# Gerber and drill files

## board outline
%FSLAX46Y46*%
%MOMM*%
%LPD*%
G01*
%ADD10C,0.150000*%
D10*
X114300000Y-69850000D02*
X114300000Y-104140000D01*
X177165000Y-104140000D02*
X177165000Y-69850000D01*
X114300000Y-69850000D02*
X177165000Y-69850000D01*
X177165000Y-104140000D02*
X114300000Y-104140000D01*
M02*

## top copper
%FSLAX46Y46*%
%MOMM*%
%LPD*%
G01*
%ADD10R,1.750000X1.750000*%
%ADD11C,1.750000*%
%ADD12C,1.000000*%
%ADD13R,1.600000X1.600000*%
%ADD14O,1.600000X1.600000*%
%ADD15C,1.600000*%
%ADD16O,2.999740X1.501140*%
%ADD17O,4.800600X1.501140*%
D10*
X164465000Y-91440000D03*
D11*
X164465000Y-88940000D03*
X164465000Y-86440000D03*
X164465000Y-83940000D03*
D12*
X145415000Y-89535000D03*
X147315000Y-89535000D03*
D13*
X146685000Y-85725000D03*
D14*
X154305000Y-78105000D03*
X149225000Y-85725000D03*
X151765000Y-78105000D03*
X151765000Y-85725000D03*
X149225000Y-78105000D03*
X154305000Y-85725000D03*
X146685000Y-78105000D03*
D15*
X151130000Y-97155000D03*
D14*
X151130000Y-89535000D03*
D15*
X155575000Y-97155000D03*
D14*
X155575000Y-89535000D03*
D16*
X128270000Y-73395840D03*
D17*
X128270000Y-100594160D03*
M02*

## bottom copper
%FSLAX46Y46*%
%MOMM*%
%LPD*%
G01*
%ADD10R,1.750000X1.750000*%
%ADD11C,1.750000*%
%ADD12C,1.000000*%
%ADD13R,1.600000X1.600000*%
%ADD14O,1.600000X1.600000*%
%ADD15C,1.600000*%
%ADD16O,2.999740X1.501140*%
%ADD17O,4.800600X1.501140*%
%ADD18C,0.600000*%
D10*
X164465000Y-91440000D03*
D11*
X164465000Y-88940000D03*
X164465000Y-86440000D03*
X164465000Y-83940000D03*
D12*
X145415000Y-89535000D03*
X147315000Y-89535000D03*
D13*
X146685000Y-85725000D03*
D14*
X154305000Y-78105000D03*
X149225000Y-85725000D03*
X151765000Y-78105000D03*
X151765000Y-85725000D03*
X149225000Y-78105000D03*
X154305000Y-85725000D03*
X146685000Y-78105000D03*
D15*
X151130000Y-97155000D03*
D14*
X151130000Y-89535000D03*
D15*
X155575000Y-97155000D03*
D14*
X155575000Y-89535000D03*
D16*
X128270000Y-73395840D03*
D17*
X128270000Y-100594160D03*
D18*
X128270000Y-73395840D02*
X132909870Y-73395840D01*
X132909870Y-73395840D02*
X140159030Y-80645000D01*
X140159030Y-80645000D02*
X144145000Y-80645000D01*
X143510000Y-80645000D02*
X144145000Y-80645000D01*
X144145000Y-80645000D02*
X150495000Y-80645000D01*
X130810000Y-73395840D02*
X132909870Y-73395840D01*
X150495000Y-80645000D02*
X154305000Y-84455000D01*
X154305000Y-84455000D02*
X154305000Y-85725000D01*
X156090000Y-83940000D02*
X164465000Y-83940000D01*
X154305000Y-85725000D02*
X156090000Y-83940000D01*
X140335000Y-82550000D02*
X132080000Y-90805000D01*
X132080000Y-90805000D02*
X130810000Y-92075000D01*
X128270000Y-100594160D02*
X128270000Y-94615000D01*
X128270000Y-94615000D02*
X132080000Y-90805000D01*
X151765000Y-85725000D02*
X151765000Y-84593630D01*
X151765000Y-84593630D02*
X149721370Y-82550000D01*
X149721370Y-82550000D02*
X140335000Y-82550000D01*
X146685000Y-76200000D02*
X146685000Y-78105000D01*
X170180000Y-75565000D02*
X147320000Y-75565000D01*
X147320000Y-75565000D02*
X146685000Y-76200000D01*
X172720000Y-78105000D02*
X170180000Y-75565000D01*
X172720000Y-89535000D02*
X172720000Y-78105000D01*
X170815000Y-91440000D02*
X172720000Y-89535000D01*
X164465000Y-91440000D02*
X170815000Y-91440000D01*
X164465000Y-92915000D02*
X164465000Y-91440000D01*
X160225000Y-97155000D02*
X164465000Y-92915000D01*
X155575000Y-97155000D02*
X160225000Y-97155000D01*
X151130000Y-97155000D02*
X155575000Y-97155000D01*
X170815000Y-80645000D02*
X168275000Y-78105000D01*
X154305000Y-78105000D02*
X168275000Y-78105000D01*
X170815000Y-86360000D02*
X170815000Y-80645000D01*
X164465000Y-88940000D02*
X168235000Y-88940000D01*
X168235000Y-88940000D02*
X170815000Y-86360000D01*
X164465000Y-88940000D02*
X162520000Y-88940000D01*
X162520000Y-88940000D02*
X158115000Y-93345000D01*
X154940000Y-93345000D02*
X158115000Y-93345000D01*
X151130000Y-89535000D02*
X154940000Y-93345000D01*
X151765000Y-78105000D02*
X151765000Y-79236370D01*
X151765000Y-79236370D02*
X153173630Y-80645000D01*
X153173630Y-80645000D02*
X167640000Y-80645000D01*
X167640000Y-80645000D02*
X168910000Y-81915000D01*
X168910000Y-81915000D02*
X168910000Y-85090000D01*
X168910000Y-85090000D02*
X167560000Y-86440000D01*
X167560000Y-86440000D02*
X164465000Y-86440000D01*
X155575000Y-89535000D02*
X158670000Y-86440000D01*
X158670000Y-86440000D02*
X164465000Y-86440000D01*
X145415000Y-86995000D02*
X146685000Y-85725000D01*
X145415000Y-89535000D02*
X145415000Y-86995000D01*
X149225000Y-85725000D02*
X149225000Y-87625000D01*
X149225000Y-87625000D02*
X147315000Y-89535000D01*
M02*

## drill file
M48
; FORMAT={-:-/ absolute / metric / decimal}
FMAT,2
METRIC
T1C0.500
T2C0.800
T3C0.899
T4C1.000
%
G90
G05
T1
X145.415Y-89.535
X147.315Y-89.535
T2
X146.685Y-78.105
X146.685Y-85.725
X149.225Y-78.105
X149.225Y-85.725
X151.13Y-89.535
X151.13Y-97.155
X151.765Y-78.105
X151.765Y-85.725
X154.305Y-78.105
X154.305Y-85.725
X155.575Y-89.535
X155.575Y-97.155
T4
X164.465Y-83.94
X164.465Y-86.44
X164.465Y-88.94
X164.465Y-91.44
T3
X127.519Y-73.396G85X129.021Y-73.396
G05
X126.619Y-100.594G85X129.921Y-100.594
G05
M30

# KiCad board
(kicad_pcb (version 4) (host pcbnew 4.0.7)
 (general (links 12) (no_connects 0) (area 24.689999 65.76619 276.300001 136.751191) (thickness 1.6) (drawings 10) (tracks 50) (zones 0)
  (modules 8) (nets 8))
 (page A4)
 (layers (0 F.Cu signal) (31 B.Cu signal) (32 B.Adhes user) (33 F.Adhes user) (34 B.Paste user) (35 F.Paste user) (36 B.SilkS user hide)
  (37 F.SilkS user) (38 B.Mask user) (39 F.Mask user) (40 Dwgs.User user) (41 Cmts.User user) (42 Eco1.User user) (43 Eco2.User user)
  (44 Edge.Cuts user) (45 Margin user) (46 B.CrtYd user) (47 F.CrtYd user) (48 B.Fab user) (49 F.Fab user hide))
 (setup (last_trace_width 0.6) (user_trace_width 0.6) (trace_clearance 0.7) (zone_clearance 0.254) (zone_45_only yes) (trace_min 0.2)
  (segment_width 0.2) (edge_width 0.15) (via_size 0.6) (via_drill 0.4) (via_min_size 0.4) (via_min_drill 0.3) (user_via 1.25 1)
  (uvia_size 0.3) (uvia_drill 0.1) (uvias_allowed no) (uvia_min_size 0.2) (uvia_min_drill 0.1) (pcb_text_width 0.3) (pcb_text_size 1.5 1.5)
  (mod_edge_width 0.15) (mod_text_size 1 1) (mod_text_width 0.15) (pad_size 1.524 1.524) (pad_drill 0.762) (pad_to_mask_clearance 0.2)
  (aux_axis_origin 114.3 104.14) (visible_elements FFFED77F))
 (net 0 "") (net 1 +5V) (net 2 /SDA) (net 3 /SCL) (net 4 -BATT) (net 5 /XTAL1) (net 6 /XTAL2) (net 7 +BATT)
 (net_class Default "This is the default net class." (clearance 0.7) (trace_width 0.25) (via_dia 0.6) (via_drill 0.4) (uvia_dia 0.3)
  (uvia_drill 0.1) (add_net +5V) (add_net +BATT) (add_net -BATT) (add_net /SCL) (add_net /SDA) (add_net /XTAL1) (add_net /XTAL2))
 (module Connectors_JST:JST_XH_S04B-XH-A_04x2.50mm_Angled (layer F.Cu) (at 164.465 91.44 90)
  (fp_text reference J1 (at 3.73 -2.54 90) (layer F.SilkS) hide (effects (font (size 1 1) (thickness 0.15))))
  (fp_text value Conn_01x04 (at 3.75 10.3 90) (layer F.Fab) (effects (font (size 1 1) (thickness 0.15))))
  (pad 1 thru_hole rect (at 0 0 90) (size 1.75 1.75) (drill 1) (layers *.Cu *.Mask F.SilkS) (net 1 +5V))
  (pad 2 thru_hole circle (at 2.5 0 90) (size 1.75 1.75) (drill 1) (layers *.Cu *.Mask F.SilkS) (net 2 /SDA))
  (pad 3 thru_hole circle (at 5 0 90) (size 1.75 1.75) (drill 1) (layers *.Cu *.Mask F.SilkS) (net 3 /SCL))
  (pad 4 thru_hole circle (at 7.5 0 90) (size 1.75 1.75) (drill 1) (layers *.Cu *.Mask F.SilkS) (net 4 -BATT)))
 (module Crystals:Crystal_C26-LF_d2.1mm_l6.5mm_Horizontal (layer F.Cu) (at 145.415 89.535)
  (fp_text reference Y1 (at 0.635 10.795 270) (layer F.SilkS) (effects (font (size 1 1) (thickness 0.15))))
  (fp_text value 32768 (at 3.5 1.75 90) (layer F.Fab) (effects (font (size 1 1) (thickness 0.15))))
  (pad 1 thru_hole circle (at 0 0) (size 1 1) (drill 0.5) (layers *.Cu *.Mask) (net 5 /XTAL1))
  (pad 2 thru_hole circle (at 1.9 0) (size 1 1) (drill 0.5) (layers *.Cu *.Mask) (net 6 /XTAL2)))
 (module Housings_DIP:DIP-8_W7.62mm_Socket (layer F.Cu) (at 146.685 85.725 90)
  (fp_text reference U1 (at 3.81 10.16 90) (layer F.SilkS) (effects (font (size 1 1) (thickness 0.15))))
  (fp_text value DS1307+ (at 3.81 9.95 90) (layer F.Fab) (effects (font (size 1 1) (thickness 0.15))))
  (pad 1 thru_hole rect (at 0 0 90) (size 1.6 1.6) (drill 0.8) (layers *.Cu *.Mask) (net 5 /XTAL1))
  (pad 5 thru_hole oval (at 7.62 7.62 90) (size 1.6 1.6) (drill 0.8) (layers *.Cu *.Mask) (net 2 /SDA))
  (pad 2 thru_hole oval (at 0 2.54 90) (size 1.6 1.6) (drill 0.8) (layers *.Cu *.Mask) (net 6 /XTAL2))
  (pad 6 thru_hole oval (at 7.62 5.08 90) (size 1.6 1.6) (drill 0.8) (layers *.Cu *.Mask) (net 3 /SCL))
  (pad 3 thru_hole oval (at 0 5.08 90) (size 1.6 1.6) (drill 0.8) (layers *.Cu *.Mask) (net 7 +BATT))
  (pad 7 thru_hole oval (at 7.62 2.54 90) (size 1.6 1.6) (drill 0.8) (layers *.Cu *.Mask))
  (pad 4 thru_hole oval (at 0 7.62 90) (size 1.6 1.6) (drill 0.8) (layers *.Cu *.Mask) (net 4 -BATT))
  (pad 8 thru_hole oval (at 7.62 0 90) (size 1.6 1.6) (drill 0.8) (layers *.Cu *.Mask) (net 1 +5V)))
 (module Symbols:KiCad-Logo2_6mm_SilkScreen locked (layer B.Cu) (at 142.24 91.44 270)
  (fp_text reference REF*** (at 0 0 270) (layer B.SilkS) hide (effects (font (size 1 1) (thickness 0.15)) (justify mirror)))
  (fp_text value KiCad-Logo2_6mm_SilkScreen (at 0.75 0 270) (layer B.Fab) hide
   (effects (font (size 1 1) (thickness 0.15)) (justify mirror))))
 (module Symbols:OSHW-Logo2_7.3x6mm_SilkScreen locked (layer B.Cu) (at 142.24 80.645 270)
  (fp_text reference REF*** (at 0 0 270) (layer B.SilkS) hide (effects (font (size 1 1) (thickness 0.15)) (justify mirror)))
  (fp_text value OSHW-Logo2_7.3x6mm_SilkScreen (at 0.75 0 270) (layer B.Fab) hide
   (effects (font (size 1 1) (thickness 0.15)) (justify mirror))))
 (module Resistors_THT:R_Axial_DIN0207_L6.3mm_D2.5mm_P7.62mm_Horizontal (layer F.Cu) (at 151.13 97.155 90)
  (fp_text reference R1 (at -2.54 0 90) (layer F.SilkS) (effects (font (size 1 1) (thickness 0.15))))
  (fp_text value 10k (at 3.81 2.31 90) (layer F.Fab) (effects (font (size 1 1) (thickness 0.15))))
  (pad 1 thru_hole circle (at 0 0 90) (size 1.6 1.6) (drill 0.8) (layers *.Cu *.Mask) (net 1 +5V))
  (pad 2 thru_hole oval (at 7.62 0 90) (size 1.6 1.6) (drill 0.8) (layers *.Cu *.Mask) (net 2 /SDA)))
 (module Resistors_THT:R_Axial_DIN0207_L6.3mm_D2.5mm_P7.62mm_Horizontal (layer F.Cu) (at 155.575 97.155 90)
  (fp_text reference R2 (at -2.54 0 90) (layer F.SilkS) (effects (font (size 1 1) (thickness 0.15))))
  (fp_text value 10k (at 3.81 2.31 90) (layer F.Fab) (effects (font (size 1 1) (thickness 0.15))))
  (pad 1 thru_hole circle (at 0 0 90) (size 1.6 1.6) (drill 0.8) (layers *.Cu *.Mask) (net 1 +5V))
  (pad 2 thru_hole oval (at 7.62 0 90) (size 1.6 1.6) (drill 0.8) (layers *.Cu *.Mask) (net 3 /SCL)))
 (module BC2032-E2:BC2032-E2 (layer F.Cu) (at 128.27 86.995 90)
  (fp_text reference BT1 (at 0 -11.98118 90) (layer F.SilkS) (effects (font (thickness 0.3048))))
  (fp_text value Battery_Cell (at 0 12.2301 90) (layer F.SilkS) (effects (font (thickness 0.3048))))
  (pad 2 thru_hole oval (at 13.59916 0 90) (size 1.50114 2.99974) (drill oval 0.89916 2.4003) (layers *.Cu *.Mask F.SilkS) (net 4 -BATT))
  (pad 1 thru_hole oval (at -13.59916 0 90) (size 1.50114 4.8006) (drill oval 0.89916 4.20116) (layers *.Cu *.Mask F.SilkS) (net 7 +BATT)))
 (gr_line (start 114.3 69.85) (end 114.3 104.14) (layer Edge.Cuts) (width 0.15))
 (gr_line (start 177.165 104.14) (end 177.165 69.85) (layer Edge.Cuts) (width 0.15))
 (gr_line (start 114.3 69.85) (end 177.165 69.85) (layer Edge.Cuts) (width 0.15))
 (gr_line (start 177.165 104.14) (end 114.3 104.14) (layer Edge.Cuts) (width 0.15))
 (segment (start 128.27 73.39584) (end 132.90987 73.39584) (width 0.6) (layer B.Cu) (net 4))
 (segment (start 132.90987 73.39584) (end 140.15903 80.645) (width 0.6) (layer B.Cu) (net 4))
 (segment (start 140.15903 80.645) (end 144.145 80.645) (width 0.6) (layer B.Cu) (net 4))
 (segment (start 143.51 80.645) (end 144.145 80.645) (width 0.6) (layer B.Cu) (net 4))
 (segment (start 144.145 80.645) (end 150.495 80.645) (width 0.6) (layer B.Cu) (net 4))
 (segment (start 130.81 73.39584) (end 132.90987 73.39584) (width 0.6) (layer B.Cu) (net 4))
 (segment (start 150.495 80.645) (end 154.305 84.455) (width 0.6) (layer B.Cu) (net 4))
 (segment (start 154.305 84.455) (end 154.305 85.725) (width 0.6) (layer B.Cu) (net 4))
 (segment (start 156.09 83.94) (end 164.465 83.94) (width 0.6) (layer B.Cu) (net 4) (status 20))
 (segment (start 154.305 85.725) (end 156.09 83.94) (width 0.6) (layer B.Cu) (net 4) (status 10))
 (segment (start 140.335 82.55) (end 132.08 90.805) (width 0.6) (layer B.Cu) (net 7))
 (segment (start 132.08 90.805) (end 130.81 92.075) (width 0.6) (layer B.Cu) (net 7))
 (segment (start 128.27 100.59416) (end 128.27 94.615) (width 0.6) (layer B.Cu) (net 7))
 (segment (start 128.27 94.615) (end 132.08 90.805) (width 0.6) (layer B.Cu) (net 7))
 (segment (start 151.765 85.725) (end 151.765 84.59363) (width 0.6) (layer B.Cu) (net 7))
 (segment (start 151.765 84.59363) (end 149.72137 82.55) (width 0.6) (layer B.Cu) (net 7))
 (segment (start 149.72137 82.55) (end 140.335 82.55) (width 0.6) (layer B.Cu) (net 7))
 (segment (start 146.685 76.2) (end 146.685 78.105) (width 0.6) (layer B.Cu) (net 1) (status 20))
 (segment (start 170.18 75.565) (end 147.32 75.565) (width 0.6) (layer B.Cu) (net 1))
 (segment (start 147.32 75.565) (end 146.685 76.2) (width 0.6) (layer B.Cu) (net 1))
 (segment (start 172.72 78.105) (end 170.18 75.565) (width 0.6) (layer B.Cu) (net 1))
 (segment (start 172.72 89.535) (end 172.72 78.105) (width 0.6) (layer B.Cu) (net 1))
 (segment (start 170.815 91.44) (end 172.72 89.535) (width 0.6) (layer B.Cu) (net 1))
 (segment (start 164.465 91.44) (end 170.815 91.44) (width 0.6) (layer B.Cu) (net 1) (status 10))
 (segment (start 164.465 92.915) (end 164.465 91.44) (width 0.6) (layer B.Cu) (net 1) (status 20))
 (segment (start 160.225 97.155) (end 164.465 92.915) (width 0.6) (layer B.Cu) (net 1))
 (segment (start 155.575 97.155) (end 160.225 97.155) (width 0.6) (layer B.Cu) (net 1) (status 10))
 (segment (start 151.13 97.155) (end 155.575 97.155) (width 0.6) (layer B.Cu) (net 1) (status 30))
 (segment (start 170.815 80.645) (end 168.275 78.105) (width 0.6) (layer B.Cu) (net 2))
 (segment (start 154.305 78.105) (end 168.275 78.105) (width 0.6) (layer B.Cu) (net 2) (status 10))
 (segment (start 170.815 86.36) (end 170.815 80.645) (width 0.6) (layer B.Cu) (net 2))
 (segment (start 164.465 88.94) (end 168.235 88.94) (width 0.6) (layer B.Cu) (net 2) (status 10))
 (segment (start 168.235 88.94) (end 170.815 86.36) (width 0.6) (layer B.Cu) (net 2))
 (segment (start 164.465 88.94) (end 162.52 88.94) (width 0.6) (layer B.Cu) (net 2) (status 10))
 (segment (start 162.52 88.94) (end 158.115 93.345) (width 0.6) (layer B.Cu) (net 2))
 (segment (start 154.94 93.345) (end 158.115 93.345) (width 0.6) (layer B.Cu) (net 2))
 (segment (start 151.13 89.535) (end 154.94 93.345) (width 0.6) (layer B.Cu) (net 2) (status 10))
 (segment (start 151.765 78.105) (end 151.765 79.23637) (width 0.6) (layer B.Cu) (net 3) (status 10))
 (segment (start 151.765 79.23637) (end 153.17363 80.645) (width 0.6) (layer B.Cu) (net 3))
 (segment (start 153.17363 80.645) (end 167.64 80.645) (width 0.6) (layer B.Cu) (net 3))
 (segment (start 167.64 80.645) (end 168.91 81.915) (width 0.6) (layer B.Cu) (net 3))
 (segment (start 168.91 81.915) (end 168.91 85.09) (width 0.6) (layer B.Cu) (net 3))
 (segment (start 168.91 85.09) (end 167.56 86.44) (width 0.6) (layer B.Cu) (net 3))
 (segment (start 167.56 86.44) (end 164.465 86.44) (width 0.6) (layer B.Cu) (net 3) (status 20))
 (segment (start 155.575 89.535) (end 158.67 86.44) (width 0.6) (layer B.Cu) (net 3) (status 10))
 (segment (start 158.67 86.44) (end 164.465 86.44) (width 0.6) (layer B.Cu) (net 3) (status 20))
 (segment (start 145.415 86.995) (end 146.685 85.725) (width 0.6) (layer B.Cu) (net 5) (status 20))
 (segment (start 145.415 89.535) (end 145.415 86.995) (width 0.6) (layer B.Cu) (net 5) (status 10))
 (segment (start 149.225 85.725) (end 149.225 87.625) (width 0.6) (layer B.Cu) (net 6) (status 10))
 (segment (start 149.225 87.625) (end 147.315 89.535) (width 0.6) (layer B.Cu) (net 6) (status 20)))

